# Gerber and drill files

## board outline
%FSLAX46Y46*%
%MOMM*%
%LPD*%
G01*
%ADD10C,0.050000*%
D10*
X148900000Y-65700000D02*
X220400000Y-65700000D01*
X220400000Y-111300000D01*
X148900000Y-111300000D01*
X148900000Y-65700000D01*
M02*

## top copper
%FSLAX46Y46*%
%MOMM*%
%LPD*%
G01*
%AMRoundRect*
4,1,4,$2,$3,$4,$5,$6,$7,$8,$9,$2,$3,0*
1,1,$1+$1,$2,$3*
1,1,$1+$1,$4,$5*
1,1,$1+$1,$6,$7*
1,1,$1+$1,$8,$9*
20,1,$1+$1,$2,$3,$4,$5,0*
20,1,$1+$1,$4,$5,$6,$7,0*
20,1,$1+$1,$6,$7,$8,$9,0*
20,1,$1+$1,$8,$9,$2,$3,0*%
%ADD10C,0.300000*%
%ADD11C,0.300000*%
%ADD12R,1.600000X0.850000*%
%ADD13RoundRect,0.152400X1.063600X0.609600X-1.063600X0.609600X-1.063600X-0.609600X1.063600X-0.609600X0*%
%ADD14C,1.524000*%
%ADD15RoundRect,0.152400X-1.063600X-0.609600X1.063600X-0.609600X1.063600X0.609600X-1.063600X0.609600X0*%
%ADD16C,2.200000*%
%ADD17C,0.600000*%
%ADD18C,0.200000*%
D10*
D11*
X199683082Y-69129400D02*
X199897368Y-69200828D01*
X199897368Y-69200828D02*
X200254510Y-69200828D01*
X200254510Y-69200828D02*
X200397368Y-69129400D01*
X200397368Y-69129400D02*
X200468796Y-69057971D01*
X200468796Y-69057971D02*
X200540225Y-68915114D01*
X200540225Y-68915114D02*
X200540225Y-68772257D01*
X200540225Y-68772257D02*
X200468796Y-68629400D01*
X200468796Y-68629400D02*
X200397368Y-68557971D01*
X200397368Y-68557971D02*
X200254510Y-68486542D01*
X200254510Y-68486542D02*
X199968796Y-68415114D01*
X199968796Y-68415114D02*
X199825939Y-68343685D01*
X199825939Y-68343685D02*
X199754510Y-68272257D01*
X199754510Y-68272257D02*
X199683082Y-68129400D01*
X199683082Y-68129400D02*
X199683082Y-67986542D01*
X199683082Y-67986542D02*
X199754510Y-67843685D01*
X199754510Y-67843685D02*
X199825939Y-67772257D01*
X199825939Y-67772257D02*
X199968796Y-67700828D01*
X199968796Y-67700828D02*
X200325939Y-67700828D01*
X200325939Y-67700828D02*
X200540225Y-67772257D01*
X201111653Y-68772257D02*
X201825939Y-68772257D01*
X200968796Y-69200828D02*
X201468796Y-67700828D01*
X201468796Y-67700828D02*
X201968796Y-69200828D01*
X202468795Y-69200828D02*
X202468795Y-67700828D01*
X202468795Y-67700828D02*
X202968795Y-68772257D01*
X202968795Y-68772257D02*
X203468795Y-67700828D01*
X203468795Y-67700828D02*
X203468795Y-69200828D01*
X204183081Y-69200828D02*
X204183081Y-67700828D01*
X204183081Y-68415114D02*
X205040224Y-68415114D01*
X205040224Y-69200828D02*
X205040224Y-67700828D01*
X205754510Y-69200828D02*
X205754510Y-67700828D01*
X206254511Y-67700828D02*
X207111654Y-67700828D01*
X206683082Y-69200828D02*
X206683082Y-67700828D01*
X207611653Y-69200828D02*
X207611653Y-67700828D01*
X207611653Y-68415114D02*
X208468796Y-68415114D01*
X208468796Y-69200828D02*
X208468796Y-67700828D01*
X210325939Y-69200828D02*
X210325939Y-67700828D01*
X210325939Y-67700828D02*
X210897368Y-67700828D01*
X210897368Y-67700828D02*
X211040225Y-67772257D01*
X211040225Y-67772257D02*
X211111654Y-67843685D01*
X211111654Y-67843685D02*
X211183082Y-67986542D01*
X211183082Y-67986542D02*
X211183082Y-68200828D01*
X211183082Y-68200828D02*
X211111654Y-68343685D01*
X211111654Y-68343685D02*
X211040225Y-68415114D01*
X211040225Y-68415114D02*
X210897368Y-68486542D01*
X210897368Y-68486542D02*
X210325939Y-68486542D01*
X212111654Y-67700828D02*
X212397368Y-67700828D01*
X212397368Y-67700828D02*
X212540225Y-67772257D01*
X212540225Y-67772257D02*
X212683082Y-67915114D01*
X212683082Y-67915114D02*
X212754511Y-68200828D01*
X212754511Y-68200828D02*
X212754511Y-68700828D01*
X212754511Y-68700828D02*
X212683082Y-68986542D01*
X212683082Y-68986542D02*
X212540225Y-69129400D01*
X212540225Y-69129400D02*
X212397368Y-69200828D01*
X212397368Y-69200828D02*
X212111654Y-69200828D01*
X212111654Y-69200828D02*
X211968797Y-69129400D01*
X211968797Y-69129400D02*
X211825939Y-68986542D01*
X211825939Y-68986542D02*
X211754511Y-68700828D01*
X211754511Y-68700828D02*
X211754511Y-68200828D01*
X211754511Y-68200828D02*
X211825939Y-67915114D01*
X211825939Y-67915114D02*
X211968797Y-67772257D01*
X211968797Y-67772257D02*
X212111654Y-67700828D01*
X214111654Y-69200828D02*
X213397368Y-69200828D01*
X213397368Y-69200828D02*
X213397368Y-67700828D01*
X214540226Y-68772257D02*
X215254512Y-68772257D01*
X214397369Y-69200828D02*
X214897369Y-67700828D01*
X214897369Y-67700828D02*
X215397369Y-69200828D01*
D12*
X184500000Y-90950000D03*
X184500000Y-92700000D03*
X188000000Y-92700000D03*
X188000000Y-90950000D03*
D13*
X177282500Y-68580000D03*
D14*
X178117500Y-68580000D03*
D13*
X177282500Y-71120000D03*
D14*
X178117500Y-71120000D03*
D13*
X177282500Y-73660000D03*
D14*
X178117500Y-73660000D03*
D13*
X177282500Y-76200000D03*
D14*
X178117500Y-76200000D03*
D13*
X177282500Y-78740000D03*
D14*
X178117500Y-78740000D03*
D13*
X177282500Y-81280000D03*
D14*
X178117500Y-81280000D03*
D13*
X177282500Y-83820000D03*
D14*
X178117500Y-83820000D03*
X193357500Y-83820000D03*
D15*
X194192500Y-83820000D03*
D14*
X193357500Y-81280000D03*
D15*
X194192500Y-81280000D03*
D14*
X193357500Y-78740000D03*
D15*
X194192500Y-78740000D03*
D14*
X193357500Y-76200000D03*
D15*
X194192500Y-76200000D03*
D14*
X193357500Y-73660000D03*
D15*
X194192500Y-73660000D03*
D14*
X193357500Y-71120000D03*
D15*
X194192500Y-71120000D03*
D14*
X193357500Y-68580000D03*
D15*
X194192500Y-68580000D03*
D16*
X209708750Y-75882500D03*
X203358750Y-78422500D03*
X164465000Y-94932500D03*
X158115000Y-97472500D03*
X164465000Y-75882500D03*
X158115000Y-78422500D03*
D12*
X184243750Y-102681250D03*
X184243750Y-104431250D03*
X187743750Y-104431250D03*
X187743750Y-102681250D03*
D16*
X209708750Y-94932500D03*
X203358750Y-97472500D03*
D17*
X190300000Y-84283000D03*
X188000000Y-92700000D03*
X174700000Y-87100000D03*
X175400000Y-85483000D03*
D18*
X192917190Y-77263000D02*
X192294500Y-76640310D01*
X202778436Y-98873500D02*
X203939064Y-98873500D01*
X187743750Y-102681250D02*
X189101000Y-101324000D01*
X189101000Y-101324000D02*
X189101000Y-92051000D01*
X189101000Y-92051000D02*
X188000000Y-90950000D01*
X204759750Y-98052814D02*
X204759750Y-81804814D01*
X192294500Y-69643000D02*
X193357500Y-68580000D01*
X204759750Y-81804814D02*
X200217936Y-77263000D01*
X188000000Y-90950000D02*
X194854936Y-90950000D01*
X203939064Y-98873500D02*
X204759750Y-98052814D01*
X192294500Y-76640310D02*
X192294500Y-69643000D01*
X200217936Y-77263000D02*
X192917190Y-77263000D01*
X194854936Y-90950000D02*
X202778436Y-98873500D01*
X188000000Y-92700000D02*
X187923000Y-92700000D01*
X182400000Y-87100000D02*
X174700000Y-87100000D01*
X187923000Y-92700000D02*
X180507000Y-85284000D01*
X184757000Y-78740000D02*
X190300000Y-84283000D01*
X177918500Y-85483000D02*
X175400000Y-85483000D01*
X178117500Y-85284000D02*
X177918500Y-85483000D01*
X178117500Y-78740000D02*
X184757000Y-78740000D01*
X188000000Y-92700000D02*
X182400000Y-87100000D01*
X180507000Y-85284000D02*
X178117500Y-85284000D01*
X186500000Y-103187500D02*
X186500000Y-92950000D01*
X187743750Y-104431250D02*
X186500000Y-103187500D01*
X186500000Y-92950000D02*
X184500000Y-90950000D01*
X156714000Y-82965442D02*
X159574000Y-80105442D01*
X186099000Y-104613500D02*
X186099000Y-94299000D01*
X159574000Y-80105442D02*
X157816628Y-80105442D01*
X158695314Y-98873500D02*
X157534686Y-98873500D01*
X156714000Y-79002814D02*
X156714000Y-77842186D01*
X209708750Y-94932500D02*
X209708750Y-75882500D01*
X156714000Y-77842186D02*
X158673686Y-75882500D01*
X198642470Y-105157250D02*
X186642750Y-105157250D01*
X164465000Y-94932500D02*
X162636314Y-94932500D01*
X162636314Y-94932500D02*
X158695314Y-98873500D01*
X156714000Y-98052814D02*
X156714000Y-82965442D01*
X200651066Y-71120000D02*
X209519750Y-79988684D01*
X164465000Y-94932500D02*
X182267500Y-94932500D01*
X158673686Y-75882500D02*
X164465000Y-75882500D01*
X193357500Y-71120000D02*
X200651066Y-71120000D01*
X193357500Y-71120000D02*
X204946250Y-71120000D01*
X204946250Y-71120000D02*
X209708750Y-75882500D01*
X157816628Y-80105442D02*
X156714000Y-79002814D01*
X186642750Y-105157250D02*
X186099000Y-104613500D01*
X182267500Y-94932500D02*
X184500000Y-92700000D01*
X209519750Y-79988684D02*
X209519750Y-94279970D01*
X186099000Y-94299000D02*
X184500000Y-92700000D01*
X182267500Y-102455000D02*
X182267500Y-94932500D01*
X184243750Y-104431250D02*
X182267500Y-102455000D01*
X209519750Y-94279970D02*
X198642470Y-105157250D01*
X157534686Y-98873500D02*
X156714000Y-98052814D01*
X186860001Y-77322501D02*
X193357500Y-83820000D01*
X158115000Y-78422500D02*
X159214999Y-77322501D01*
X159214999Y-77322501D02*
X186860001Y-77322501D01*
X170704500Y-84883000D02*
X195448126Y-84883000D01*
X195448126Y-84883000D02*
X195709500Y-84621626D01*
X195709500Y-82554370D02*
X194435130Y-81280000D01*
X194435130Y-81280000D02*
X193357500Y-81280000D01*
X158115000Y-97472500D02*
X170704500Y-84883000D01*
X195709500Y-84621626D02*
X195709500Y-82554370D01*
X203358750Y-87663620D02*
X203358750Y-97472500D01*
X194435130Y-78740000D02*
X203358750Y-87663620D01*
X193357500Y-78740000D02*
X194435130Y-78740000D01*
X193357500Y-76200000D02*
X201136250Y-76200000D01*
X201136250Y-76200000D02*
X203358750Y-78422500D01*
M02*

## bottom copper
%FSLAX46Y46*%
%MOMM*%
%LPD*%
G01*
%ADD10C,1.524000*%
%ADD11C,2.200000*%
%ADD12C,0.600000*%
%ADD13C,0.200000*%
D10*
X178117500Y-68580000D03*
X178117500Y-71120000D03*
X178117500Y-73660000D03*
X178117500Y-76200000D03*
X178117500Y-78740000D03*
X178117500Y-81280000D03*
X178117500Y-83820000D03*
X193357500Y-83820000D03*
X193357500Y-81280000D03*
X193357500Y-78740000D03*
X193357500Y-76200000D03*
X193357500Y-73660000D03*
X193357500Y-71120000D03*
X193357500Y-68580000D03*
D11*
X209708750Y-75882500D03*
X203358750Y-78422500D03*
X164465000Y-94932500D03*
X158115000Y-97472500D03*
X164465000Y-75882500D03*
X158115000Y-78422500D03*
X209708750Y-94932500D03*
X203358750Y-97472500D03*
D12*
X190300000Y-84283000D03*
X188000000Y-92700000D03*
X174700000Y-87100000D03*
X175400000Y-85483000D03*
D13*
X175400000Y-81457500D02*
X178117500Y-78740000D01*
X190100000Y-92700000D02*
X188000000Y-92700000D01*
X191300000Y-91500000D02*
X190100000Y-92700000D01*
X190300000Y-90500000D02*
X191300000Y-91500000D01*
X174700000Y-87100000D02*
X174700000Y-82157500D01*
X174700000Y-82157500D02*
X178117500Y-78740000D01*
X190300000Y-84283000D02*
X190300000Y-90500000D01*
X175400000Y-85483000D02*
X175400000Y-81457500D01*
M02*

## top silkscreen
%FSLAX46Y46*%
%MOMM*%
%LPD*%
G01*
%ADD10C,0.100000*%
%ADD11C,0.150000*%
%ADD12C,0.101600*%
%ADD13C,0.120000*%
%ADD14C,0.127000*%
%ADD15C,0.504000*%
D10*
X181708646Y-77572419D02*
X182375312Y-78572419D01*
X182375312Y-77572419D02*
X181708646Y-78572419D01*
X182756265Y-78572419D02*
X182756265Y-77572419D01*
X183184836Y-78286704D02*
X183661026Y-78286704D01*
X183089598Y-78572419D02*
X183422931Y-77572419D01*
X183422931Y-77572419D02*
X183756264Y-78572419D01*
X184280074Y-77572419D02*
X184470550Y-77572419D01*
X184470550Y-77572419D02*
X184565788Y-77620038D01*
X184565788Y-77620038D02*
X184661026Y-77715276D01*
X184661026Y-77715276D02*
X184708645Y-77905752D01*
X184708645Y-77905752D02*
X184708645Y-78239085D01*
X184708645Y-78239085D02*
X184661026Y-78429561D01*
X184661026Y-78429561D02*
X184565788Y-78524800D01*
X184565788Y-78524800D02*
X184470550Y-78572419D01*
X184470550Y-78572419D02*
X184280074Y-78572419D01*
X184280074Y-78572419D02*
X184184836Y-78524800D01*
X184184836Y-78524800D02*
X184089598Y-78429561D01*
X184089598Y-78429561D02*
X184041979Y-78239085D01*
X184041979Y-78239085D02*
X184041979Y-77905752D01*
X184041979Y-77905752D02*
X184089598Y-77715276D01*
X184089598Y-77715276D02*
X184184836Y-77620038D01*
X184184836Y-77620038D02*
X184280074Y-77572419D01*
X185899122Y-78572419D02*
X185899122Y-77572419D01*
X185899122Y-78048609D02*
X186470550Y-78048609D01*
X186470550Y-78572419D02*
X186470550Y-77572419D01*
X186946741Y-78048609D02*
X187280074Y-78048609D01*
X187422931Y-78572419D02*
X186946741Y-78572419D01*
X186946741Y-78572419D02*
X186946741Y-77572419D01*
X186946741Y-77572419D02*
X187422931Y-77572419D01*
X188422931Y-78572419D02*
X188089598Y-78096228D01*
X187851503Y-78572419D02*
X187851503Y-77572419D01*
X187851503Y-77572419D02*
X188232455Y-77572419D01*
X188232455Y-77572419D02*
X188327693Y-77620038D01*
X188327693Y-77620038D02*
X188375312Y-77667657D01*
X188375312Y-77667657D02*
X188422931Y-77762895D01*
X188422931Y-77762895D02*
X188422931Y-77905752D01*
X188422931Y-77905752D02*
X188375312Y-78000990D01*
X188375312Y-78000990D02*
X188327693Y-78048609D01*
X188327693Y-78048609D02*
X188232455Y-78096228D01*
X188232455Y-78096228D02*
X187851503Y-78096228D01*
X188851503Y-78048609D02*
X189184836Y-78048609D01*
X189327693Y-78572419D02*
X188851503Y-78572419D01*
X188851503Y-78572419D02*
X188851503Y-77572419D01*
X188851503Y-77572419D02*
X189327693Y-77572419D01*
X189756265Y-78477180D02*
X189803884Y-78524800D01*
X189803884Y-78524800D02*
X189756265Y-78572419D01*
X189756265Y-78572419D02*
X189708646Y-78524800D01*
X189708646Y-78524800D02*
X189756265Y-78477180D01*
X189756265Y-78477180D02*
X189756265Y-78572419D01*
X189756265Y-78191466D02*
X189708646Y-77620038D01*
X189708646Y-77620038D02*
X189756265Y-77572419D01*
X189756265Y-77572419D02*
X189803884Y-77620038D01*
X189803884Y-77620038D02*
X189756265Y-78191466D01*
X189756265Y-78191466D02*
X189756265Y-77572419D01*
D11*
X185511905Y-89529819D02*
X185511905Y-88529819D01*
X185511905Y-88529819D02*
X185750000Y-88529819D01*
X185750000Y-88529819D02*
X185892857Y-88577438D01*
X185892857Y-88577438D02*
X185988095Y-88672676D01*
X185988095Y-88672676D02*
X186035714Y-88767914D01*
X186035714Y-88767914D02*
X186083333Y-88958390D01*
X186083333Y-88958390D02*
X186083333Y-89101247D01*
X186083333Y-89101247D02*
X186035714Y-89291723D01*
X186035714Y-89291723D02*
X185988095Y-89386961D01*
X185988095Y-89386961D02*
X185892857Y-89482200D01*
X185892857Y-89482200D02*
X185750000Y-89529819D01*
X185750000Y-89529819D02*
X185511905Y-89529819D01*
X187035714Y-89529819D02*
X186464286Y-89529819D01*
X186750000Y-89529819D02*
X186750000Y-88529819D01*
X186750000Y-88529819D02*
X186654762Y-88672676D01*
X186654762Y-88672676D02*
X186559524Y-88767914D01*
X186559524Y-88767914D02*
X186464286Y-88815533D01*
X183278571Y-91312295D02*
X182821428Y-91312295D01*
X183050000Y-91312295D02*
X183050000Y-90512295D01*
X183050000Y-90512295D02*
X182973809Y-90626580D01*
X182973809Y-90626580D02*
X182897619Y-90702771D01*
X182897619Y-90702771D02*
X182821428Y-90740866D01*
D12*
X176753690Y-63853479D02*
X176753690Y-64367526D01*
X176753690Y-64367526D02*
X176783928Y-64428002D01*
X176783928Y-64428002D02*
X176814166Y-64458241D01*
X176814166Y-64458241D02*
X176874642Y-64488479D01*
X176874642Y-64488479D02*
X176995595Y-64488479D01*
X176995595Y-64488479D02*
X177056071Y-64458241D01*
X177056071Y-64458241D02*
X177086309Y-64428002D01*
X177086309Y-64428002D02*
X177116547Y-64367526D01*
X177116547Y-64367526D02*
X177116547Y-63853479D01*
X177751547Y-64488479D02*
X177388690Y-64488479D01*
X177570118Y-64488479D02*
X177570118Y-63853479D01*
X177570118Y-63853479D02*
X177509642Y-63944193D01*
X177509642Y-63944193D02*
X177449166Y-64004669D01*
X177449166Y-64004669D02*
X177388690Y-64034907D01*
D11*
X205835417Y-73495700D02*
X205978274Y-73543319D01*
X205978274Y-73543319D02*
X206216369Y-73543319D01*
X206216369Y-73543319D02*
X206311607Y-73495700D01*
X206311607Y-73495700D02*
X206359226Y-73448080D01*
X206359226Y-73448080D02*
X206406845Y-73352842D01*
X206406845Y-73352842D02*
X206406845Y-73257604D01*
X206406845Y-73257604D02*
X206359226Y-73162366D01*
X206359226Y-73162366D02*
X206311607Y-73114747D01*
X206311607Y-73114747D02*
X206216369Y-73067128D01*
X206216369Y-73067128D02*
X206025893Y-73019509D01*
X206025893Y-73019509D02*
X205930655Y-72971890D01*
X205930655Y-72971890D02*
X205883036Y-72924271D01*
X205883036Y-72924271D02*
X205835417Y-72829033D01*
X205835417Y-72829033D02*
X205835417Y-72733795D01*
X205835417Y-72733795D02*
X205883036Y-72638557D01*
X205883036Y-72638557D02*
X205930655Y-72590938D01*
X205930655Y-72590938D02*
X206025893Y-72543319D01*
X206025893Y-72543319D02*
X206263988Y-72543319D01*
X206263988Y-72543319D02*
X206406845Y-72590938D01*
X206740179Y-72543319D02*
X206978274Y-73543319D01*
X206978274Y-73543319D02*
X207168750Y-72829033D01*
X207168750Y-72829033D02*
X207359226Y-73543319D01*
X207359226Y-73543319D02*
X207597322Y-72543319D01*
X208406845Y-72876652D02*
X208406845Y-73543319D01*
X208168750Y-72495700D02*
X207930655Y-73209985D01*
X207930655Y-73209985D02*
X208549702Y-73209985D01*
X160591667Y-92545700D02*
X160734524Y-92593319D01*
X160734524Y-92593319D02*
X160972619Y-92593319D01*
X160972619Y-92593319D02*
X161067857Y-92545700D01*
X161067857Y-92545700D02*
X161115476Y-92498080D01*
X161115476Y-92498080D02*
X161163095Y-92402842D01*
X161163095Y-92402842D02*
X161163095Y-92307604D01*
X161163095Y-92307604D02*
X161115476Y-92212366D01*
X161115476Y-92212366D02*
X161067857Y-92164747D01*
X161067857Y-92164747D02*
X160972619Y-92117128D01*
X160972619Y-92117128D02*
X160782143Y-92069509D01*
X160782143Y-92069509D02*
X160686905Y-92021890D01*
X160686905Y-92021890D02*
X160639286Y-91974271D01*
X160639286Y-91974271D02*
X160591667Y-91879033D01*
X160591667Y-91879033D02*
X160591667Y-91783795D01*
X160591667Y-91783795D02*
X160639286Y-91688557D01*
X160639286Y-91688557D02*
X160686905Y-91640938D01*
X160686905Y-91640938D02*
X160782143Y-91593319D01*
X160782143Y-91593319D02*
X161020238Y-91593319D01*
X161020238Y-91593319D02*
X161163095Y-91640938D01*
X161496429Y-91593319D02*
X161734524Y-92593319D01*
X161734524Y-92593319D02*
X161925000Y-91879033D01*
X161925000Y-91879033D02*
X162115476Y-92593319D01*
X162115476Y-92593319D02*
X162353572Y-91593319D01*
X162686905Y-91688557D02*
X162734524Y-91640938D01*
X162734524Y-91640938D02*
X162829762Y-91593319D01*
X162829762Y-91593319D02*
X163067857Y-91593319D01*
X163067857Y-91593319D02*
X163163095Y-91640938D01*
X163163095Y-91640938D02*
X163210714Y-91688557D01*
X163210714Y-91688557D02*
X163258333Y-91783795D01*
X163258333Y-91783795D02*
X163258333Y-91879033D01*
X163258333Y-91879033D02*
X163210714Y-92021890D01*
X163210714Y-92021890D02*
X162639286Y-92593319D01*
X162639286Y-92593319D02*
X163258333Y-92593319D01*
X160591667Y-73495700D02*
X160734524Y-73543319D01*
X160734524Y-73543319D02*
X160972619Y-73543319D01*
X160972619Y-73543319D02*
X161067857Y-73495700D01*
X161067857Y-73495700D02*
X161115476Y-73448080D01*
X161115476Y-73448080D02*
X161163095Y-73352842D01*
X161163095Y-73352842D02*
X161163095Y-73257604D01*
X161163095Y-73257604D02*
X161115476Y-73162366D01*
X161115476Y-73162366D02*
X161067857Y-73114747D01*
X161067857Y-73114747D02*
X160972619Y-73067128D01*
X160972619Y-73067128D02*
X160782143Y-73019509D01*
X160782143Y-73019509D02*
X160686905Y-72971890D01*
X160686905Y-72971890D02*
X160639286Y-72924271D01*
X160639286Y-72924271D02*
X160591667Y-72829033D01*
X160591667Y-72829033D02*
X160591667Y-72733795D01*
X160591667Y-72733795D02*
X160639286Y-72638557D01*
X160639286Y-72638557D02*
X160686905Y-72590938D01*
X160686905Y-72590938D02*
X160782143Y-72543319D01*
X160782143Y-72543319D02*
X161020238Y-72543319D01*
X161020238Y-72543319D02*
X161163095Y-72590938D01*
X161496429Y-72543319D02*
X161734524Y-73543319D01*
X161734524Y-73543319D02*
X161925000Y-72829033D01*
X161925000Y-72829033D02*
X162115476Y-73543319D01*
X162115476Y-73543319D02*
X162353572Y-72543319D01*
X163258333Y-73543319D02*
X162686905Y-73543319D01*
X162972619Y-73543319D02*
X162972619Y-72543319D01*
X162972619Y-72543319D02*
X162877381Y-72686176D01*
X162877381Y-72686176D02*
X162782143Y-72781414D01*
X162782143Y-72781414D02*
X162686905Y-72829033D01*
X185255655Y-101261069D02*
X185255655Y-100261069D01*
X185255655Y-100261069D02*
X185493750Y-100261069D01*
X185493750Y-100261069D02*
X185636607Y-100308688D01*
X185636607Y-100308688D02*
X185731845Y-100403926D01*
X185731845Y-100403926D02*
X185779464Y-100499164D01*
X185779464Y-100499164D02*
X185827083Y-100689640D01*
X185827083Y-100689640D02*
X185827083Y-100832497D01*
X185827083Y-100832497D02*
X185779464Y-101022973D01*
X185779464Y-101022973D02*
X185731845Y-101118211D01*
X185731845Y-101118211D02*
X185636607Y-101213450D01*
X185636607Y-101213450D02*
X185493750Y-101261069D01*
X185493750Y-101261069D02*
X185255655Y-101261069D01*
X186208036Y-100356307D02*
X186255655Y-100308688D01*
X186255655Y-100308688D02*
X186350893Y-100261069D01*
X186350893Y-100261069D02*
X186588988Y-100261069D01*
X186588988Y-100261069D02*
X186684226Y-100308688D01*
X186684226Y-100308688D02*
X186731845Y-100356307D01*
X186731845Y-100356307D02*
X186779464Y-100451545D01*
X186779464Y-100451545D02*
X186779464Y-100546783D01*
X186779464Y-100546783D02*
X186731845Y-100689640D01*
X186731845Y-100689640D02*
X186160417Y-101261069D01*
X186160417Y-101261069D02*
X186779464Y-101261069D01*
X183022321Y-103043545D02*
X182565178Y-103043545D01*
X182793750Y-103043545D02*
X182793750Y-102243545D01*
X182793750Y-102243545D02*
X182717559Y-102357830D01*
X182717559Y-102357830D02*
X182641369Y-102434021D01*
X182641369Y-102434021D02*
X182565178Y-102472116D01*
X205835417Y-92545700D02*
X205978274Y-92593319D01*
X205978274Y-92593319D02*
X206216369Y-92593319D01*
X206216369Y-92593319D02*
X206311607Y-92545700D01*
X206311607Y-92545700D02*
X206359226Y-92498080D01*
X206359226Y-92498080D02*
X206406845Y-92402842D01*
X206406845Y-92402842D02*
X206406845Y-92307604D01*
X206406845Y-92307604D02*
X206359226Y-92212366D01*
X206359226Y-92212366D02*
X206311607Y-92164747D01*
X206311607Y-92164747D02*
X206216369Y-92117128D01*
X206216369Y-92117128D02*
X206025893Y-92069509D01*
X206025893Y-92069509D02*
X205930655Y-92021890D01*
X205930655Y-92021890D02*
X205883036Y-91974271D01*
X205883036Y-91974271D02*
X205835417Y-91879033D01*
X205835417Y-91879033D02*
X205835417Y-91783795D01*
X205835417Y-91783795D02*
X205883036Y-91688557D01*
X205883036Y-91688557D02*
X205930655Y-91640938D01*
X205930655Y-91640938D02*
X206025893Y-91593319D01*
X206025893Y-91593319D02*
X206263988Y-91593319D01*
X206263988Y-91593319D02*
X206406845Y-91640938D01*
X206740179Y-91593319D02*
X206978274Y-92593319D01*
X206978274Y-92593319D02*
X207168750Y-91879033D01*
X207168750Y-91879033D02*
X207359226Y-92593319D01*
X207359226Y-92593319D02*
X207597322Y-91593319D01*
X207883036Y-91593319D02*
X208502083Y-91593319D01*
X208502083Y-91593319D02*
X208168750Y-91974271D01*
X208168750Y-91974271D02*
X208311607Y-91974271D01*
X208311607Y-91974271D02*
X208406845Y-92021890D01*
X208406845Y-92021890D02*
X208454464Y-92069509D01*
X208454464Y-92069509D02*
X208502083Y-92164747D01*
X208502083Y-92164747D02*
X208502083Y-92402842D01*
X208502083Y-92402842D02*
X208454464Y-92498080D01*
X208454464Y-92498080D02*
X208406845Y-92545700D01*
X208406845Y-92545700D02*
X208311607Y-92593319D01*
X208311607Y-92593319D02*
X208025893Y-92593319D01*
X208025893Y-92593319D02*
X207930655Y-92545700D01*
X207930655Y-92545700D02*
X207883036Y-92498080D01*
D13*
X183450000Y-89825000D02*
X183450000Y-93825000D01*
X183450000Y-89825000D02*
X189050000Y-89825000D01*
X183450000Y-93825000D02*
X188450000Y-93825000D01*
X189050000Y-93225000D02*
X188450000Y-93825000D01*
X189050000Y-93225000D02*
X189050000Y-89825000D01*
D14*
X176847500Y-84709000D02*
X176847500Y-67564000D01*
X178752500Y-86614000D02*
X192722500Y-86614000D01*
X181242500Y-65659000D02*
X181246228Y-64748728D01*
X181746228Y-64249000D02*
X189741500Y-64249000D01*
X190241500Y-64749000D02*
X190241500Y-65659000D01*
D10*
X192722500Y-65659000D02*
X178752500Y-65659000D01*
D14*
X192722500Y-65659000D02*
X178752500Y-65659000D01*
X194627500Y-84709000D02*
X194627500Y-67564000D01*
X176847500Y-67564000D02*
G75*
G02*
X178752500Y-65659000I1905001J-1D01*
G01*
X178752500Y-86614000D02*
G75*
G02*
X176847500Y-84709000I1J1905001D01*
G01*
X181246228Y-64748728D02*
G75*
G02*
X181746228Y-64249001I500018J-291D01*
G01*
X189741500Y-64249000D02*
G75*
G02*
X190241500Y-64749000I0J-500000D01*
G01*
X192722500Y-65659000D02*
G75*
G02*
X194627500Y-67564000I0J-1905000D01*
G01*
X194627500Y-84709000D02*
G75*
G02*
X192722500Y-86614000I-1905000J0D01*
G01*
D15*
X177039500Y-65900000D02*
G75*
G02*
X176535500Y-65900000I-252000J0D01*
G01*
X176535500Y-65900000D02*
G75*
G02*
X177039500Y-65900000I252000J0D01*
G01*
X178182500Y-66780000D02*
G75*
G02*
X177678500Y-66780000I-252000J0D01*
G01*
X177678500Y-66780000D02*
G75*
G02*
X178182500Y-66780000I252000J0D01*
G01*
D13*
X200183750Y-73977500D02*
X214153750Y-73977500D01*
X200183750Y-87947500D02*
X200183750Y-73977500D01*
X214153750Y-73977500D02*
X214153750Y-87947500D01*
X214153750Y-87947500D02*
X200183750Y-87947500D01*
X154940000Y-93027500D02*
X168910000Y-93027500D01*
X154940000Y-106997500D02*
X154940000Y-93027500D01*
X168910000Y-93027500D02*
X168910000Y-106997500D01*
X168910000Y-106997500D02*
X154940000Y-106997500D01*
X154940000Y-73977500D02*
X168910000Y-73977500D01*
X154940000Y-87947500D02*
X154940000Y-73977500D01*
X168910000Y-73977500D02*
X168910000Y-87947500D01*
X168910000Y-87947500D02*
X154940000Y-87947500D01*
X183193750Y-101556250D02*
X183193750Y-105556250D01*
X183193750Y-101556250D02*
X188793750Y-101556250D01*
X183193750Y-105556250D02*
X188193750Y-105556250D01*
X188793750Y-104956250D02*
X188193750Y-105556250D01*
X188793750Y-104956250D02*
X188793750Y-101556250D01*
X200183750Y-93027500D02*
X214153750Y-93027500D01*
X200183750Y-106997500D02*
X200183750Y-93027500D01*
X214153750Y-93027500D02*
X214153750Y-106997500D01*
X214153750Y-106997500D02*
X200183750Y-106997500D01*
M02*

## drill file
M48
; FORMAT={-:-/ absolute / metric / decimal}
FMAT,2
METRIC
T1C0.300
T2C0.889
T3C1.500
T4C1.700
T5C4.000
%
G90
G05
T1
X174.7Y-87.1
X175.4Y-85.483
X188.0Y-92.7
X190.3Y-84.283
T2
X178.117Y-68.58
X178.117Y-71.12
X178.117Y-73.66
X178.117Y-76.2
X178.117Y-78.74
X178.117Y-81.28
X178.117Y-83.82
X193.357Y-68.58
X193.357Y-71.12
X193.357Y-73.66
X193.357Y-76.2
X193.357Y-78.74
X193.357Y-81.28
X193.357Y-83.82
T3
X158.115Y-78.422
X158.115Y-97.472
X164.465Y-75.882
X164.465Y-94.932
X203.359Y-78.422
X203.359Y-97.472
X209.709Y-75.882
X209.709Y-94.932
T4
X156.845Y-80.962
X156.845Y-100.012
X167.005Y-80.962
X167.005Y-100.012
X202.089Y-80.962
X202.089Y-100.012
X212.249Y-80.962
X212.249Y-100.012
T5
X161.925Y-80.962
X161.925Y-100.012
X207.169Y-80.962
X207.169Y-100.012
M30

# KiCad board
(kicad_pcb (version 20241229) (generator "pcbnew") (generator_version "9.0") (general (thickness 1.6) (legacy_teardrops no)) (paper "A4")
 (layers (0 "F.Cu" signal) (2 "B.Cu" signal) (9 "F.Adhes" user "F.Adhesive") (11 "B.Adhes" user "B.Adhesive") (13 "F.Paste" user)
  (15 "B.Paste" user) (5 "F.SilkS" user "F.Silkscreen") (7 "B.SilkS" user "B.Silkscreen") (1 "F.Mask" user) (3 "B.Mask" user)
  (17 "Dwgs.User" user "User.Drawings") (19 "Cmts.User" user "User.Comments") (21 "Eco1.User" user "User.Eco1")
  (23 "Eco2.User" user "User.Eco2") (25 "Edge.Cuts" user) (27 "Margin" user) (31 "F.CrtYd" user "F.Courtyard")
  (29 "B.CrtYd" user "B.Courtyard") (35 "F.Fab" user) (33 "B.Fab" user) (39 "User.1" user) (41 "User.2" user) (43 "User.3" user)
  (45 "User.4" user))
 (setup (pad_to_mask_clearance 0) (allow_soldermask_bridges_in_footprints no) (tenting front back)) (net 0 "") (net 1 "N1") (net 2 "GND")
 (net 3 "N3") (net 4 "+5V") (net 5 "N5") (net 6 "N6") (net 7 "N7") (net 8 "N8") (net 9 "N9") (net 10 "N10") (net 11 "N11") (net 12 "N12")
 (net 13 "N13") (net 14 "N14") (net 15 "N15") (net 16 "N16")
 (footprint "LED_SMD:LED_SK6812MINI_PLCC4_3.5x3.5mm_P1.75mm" (layer "F.Cu") (at 186.25 91.825)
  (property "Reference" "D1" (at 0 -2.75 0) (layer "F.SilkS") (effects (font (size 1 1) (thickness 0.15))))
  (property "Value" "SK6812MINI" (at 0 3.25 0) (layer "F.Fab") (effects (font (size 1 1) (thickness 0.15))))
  (fp_line (start -2.8 -2) (end -2.8 2) (stroke (width 0.12) (type default)) (layer "F.SilkS"))
  (fp_line (start -2.8 -2) (end 2.8 -2) (stroke (width 0.12) (type solid)) (layer "F.SilkS"))
  (fp_line (start -2.8 2) (end 2.2 2) (stroke (width 0.12) (type solid)) (layer "F.SilkS"))
  (fp_line (start 2.8 1.4) (end 2.2 2) (stroke (width 0.12) (type default)) (layer "F.SilkS"))
  (fp_line (start 2.8 1.4) (end 2.8 -2) (stroke (width 0.12) (type solid)) (layer "F.SilkS"))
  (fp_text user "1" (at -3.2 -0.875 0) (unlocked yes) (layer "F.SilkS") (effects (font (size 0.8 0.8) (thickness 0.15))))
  (pad "1" smd rect (at -1.75 -0.875) (size 1.6 0.85) (layers "F.Cu" "F.Mask" "F.Paste") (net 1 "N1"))
  (pad "2" smd rect (at -1.75 0.875) (size 1.6 0.85) (layers "F.Cu" "F.Mask" "F.Paste") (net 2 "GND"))
  (pad "3" smd rect (at 1.75 0.875) (size 1.6 0.85) (layers "F.Cu" "F.Mask" "F.Paste") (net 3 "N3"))
  (pad "4" smd rect (at 1.75 -0.875) (size 1.6 0.85) (layers "F.Cu" "F.Mask" "F.Paste") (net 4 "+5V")))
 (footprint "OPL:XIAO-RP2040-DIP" (layer "F.Cu") (at 185.7375 76.2)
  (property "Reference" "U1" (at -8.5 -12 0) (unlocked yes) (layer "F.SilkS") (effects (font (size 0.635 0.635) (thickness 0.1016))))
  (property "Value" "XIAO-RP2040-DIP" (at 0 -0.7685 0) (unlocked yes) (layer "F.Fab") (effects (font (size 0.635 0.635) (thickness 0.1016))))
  (fp_line (start -8.89 8.509) (end -8.89 -8.636) (stroke (width 0.127) (type solid)) (layer "F.SilkS"))
  (fp_line (start -6.985 10.414) (end 6.985 10.414) (stroke (width 0.127) (type solid)) (layer "F.SilkS"))
  (fp_line (start -4.495 -10.541) (end -4.491272 -11.451272) (stroke (width 0.127) (type solid)) (layer "F.SilkS"))
  (fp_line (start -3.991272 -11.951) (end 4.004 -11.951) (stroke (width 0.127) (type solid)) (layer "F.SilkS"))
  (fp_line (start 4.504 -11.451) (end 4.504 -10.541) (stroke (width 0.127) (type solid)) (layer "F.SilkS"))
  (fp_line (start 6.985 -10.541) (end -6.985 -10.541) (stroke (width 0.1) (type solid)) (layer "F.SilkS"))
  (fp_line (start 6.985 -10.541) (end -6.985 -10.541) (stroke (width 0.127) (type solid)) (layer "F.SilkS"))
  (fp_line (start 8.89 8.509) (end 8.89 -8.636) (stroke (width 0.127) (type solid)) (layer "F.SilkS"))
  (fp_arc (start -8.89 -8.636) (mid -8.332038 -9.983038) (end -6.985 -10.541) (stroke (width 0.127) (type solid)) (layer "F.SilkS"))
  (fp_arc (start -6.985 10.414) (mid -8.332038 9.856038) (end -8.89 8.509) (stroke (width 0.127) (type solid)) (layer "F.SilkS"))
  (fp_arc (start -4.491272 -11.451272) (mid -4.344728 -11.80464) (end -3.991272 -11.951) (stroke (width 0.127) (type default))
   (layer "F.SilkS"))
  (fp_arc (start 4.004 -11.951) (mid 4.357553 -11.804553) (end 4.504 -11.451) (stroke (width 0.127) (type default)) (layer "F.SilkS"))
  (fp_arc (start 6.985 -10.541) (mid 8.332038 -9.983038) (end 8.89 -8.636) (stroke (width 0.127) (type solid)) (layer "F.SilkS"))
  (fp_arc (start 8.89 8.509) (mid 8.332038 9.856038) (end 6.985 10.414) (stroke (width 0.127) (type solid)) (layer "F.SilkS"))
  (fp_circle (center -8.95 -10.3) (end -8.95 -10.554) (stroke (width 0.5) (type solid)) (fill yes) (layer "F.SilkS"))
  (fp_circle (center -7.807 -9.42) (end -7.807 -9.674) (stroke (width 0.5) (type solid)) (fill yes) (layer "F.SilkS"))
  (pad "1" smd roundrect (at -8.455 -7.62 180) (size 2.432 1.524) (layers "F.Cu" "F.Mask") (roundrect_rratio 0.1) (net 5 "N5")
   (thermal_bridge_angle 45))
  (pad "1" thru_hole circle (at -7.62 -7.62 180) (size 1.524 1.524) (drill 0.889) (layers "*.Cu" "*.Mask") (remove_unused_layers no)
   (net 5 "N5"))
  (pad "2" smd roundrect (at -8.455 -5.08 180) (size 2.432 1.524) (layers "F.Cu" "F.Mask") (roundrect_rratio 0.1) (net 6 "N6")
   (thermal_bridge_angle 45))
  (pad "2" thru_hole circle (at -7.62 -5.08 180) (size 1.524 1.524) (drill 0.889) (layers "*.Cu" "*.Mask") (remove_unused_layers no)
   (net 6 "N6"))
  (pad "3" smd roundrect (at -8.455 -2.54 180) (size 2.432 1.524) (layers "F.Cu" "F.Mask") (roundrect_rratio 0.1) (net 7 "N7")
   (thermal_bridge_angle 45))
  (pad "3" thru_hole circle (at -7.62 -2.54 180) (size 1.524 1.524) (drill 0.889) (layers "*.Cu" "*.Mask") (remove_unused_layers no)
   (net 7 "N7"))
  (pad "4" smd roundrect (at -8.455 0 180) (size 2.432 1.524) (layers "F.Cu" "F.Mask") (roundrect_rratio 0.1) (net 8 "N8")
   (thermal_bridge_angle 45))
  (pad "4" thru_hole circle (at -7.62 0 180) (size 1.524 1.524) (drill 0.889) (layers "*.Cu" "*.Mask") (remove_unused_layers no)
   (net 8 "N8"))
  (pad "5" smd roundrect (at -8.455 2.54 180) (size 2.432 1.524) (layers "F.Cu" "F.Mask") (roundrect_rratio 0.1) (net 3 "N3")
   (thermal_bridge_angle 45))
  (pad "5" thru_hole circle (at -7.62 2.54 180) (size 1.524 1.524) (drill 0.889) (layers "*.Cu" "*.Mask") (remove_unused_layers no)
   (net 3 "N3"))
  (pad "6" smd roundrect (at -8.455 5.08 180) (size 2.432 1.524) (layers "F.Cu" "F.Mask") (roundrect_rratio 0.1) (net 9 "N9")
   (thermal_bridge_angle 45))
  (pad "6" thru_hole circle (at -7.62 5.08 180) (size 1.524 1.524) (drill 0.889) (layers "*.Cu" "*.Mask") (remove_unused_layers no)
   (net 9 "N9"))
  (pad "7" smd roundrect (at -8.455 7.62 180) (size 2.432 1.524) (layers "F.Cu" "F.Mask") (roundrect_rratio 0.1) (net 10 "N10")
   (thermal_bridge_angle 45))
  (pad "7" thru_hole circle (at -7.62 7.62 180) (size 1.524 1.524) (drill 0.889) (layers "*.Cu" "*.Mask") (remove_unused_layers no)
   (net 10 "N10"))
  (pad "8" thru_hole circle (at 7.62 7.62) (size 1.524 1.524) (drill 0.889) (layers "*.Cu" "*.Mask") (remove_unused_layers no)
   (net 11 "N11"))
  (pad "8" smd roundrect (at 8.455 7.62) (size 2.432 1.524) (layers "F.Cu" "F.Mask") (roundrect_rratio 0.1) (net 11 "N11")
   (thermal_bridge_angle 45))
  (pad "9" thru_hole circle (at 7.62 5.08) (size 1.524 1.524) (drill 0.889) (layers "*.Cu" "*.Mask") (remove_unused_layers no)
   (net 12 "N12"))
  (pad "9" smd roundrect (at 8.455 5.08) (size 2.432 1.524) (layers "F.Cu" "F.Mask") (roundrect_rratio 0.1) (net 12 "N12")
   (thermal_bridge_angle 45))
  (pad "10" thru_hole circle (at 7.62 2.54) (size 1.524 1.524) (drill 0.889) (layers "*.Cu" "*.Mask") (remove_unused_layers no)
   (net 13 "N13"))
  (pad "10" smd roundrect (at 8.455 2.54) (size 2.432 1.524) (layers "F.Cu" "F.Mask") (roundrect_rratio 0.1) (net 13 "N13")
   (thermal_bridge_angle 45))
  (pad "11" thru_hole circle (at 7.62 0) (size 1.524 1.524) (drill 0.889) (layers "*.Cu" "*.Mask") (remove_unused_layers no) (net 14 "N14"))
  (pad "11" smd roundrect (at 8.455 0) (size 2.432 1.524) (layers "F.Cu" "F.Mask") (roundrect_rratio 0.1) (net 14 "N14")
   (thermal_bridge_angle 45))
  (pad "12" thru_hole circle (at 7.62 -2.54) (size 1.524 1.524) (drill 0.889) (layers "*.Cu" "*.Mask") (remove_unused_layers no)
   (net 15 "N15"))
  (pad "12" smd roundrect (at 8.455 -2.54) (size 2.432 1.524) (layers "F.Cu" "F.Mask") (roundrect_rratio 0.1) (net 15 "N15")
   (thermal_bridge_angle 45))
  (pad "13" thru_hole circle (at 7.62 -5.08) (size 1.524 1.524) (drill 0.889) (layers "*.Cu" "*.Mask") (remove_unused_layers no)
   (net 2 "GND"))
  (pad "13" smd roundrect (at 8.455 -5.08) (size 2.432 1.524) (layers "F.Cu" "F.Mask") (roundrect_rratio 0.1) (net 2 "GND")
   (thermal_bridge_angle 45))
  (pad "14" thru_hole circle (at 7.62 -7.62) (size 1.524 1.524) (drill 0.889) (layers "*.Cu" "*.Mask") (remove_unused_layers no)
   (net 4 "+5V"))
  (pad "14" smd roundrect (at 8.455 -7.62) (size 2.432 1.524) (layers "F.Cu" "F.Mask") (roundrect_rratio 0.1) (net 4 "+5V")
   (thermal_bridge_angle 45)))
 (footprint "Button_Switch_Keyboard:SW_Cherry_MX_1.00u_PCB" (layer "F.Cu") (at 209.70875 75.8825)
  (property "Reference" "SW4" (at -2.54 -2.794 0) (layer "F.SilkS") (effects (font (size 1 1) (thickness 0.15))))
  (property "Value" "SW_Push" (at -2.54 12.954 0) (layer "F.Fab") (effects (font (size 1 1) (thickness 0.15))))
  (fp_line (start -9.525 -1.905) (end 4.445 -1.905) (stroke (width 0.12) (type solid)) (layer "F.SilkS"))
  (fp_line (start -9.525 12.065) (end -9.525 -1.905) (stroke (width 0.12) (type solid)) (layer "F.SilkS"))
  (fp_line (start 4.445 -1.905) (end 4.445 12.065) (stroke (width 0.12) (type solid)) (layer "F.SilkS"))
  (fp_line (start 4.445 12.065) (end -9.525 12.065) (stroke (width 0.12) (type solid)) (layer "F.SilkS"))
  (pad "" np_thru_hole circle (at -7.62 5.08) (size 1.7 1.7) (drill 1.7) (layers "*.Cu" "*.Mask"))
  (pad "" np_thru_hole circle (at -2.54 5.08) (size 4 4) (drill 4) (layers "*.Cu" "*.Mask"))
  (pad "" np_thru_hole circle (at 2.54 5.08) (size 1.7 1.7) (drill 1.7) (layers "*.Cu" "*.Mask"))
  (pad "1" thru_hole circle (at 0 0) (size 2.2 2.2) (drill 1.5) (layers "*.Cu" "*.Mask") (remove_unused_layers no) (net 2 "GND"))
  (pad "2" thru_hole circle (at -6.35 2.54) (size 2.2 2.2) (drill 1.5) (layers "*.Cu" "*.Mask") (remove_unused_layers no) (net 14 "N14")))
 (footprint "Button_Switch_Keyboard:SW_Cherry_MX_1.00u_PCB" (layer "F.Cu") (at 164.465 94.9325)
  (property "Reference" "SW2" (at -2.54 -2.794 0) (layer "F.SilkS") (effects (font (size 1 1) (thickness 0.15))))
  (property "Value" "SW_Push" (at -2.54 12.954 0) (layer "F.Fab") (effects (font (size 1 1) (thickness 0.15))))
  (fp_line (start -9.525 -1.905) (end 4.445 -1.905) (stroke (width 0.12) (type solid)) (layer "F.SilkS"))
  (fp_line (start -9.525 12.065) (end -9.525 -1.905) (stroke (width 0.12) (type solid)) (layer "F.SilkS"))
  (fp_line (start 4.445 -1.905) (end 4.445 12.065) (stroke (width 0.12) (type solid)) (layer "F.SilkS"))
  (fp_line (start 4.445 12.065) (end -9.525 12.065) (stroke (width 0.12) (type solid)) (layer "F.SilkS"))
  (pad "" np_thru_hole circle (at -7.62 5.08) (size 1.7 1.7) (drill 1.7) (layers "*.Cu" "*.Mask"))
  (pad "" np_thru_hole circle (at -2.54 5.08) (size 4 4) (drill 4) (layers "*.Cu" "*.Mask"))
  (pad "" np_thru_hole circle (at 2.54 5.08) (size 1.7 1.7) (drill 1.7) (layers "*.Cu" "*.Mask"))
  (pad "1" thru_hole circle (at 0 0) (size 2.2 2.2) (drill 1.5) (layers "*.Cu" "*.Mask") (remove_unused_layers no) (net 2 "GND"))
  (pad "2" thru_hole circle (at -6.35 2.54) (size 2.2 2.2) (drill 1.5) (layers "*.Cu" "*.Mask") (remove_unused_layers no) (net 12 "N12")))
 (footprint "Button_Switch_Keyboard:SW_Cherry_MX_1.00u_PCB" (layer "F.Cu") (at 164.465 75.8825)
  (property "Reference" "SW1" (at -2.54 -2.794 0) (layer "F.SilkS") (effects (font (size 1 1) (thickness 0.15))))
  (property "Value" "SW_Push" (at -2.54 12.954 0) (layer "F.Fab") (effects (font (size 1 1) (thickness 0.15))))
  (fp_line (start -9.525 -1.905) (end 4.445 -1.905) (stroke (width 0.12) (type solid)) (layer "F.SilkS"))
  (fp_line (start -9.525 12.065) (end -9.525 -1.905) (stroke (width 0.12) (type solid)) (layer "F.SilkS"))
  (fp_line (start 4.445 -1.905) (end 4.445 12.065) (stroke (width 0.12) (type solid)) (layer "F.SilkS"))
  (fp_line (start 4.445 12.065) (end -9.525 12.065) (stroke (width 0.12) (type solid)) (layer "F.SilkS"))
  (pad "" np_thru_hole circle (at -7.62 5.08) (size 1.7 1.7) (drill 1.7) (layers "*.Cu" "*.Mask"))
  (pad "" np_thru_hole circle (at -2.54 5.08) (size 4 4) (drill 4) (layers "*.Cu" "*.Mask"))
  (pad "" np_thru_hole circle (at 2.54 5.08) (size 1.7 1.7) (drill 1.7) (layers "*.Cu" "*.Mask"))
  (pad "1" thru_hole circle (at 0 0) (size 2.2 2.2) (drill 1.5) (layers "*.Cu" "*.Mask") (remove_unused_layers no) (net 2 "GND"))
  (pad "2" thru_hole circle (at -6.35 2.54) (size 2.2 2.2) (drill 1.5) (layers "*.Cu" "*.Mask") (remove_unused_layers no) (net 11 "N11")))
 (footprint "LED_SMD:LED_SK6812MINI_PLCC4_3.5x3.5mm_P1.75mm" (layer "F.Cu") (at 185.99375 103.55625)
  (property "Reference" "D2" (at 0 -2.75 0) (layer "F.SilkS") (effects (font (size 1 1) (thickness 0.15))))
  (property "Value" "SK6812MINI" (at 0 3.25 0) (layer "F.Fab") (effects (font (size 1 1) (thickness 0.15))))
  (fp_line (start -2.8 -2) (end -2.8 2) (stroke (width 0.12) (type default)) (layer "F.SilkS"))
  (fp_line (start -2.8 -2) (end 2.8 -2) (stroke (width 0.12) (type solid)) (layer "F.SilkS"))
  (fp_line (start -2.8 2) (end 2.2 2) (stroke (width 0.12) (type solid)) (layer "F.SilkS"))
  (fp_line (start 2.8 1.4) (end 2.2 2) (stroke (width 0.12) (type default)) (layer "F.SilkS"))
  (fp_line (start 2.8 1.4) (end 2.8 -2) (stroke (width 0.12) (type solid)) (layer "F.SilkS"))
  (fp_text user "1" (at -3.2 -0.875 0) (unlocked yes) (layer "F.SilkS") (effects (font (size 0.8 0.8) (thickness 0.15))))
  (pad "1" smd rect (at -1.75 -0.875) (size 1.6 0.85) (layers "F.Cu" "F.Mask" "F.Paste") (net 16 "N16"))
  (pad "2" smd rect (at -1.75 0.875) (size 1.6 0.85) (layers "F.Cu" "F.Mask" "F.Paste") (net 2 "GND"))
  (pad "3" smd rect (at 1.75 0.875) (size 1.6 0.85) (layers "F.Cu" "F.Mask" "F.Paste") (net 1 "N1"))
  (pad "4" smd rect (at 1.75 -0.875) (size 1.6 0.85) (layers "F.Cu" "F.Mask" "F.Paste") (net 4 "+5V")))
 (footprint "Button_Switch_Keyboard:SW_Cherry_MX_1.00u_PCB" (layer "F.Cu") (at 209.70875 94.9325)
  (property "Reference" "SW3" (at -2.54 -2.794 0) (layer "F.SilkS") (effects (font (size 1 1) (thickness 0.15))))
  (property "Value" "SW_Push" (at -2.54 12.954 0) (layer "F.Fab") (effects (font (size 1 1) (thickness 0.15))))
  (fp_line (start -9.525 -1.905) (end 4.445 -1.905) (stroke (width 0.12) (type solid)) (layer "F.SilkS"))
  (fp_line (start -9.525 12.065) (end -9.525 -1.905) (stroke (width 0.12) (type solid)) (layer "F.SilkS"))
  (fp_line (start 4.445 -1.905) (end 4.445 12.065) (stroke (width 0.12) (type solid)) (layer "F.SilkS"))
  (fp_line (start 4.445 12.065) (end -9.525 12.065) (stroke (width 0.12) (type solid)) (layer "F.SilkS"))
  (pad "" np_thru_hole circle (at -7.62 5.08) (size 1.7 1.7) (drill 1.7) (layers "*.Cu" "*.Mask"))
  (pad "" np_thru_hole circle (at -2.54 5.08) (size 4 4) (drill 4) (layers "*.Cu" "*.Mask"))
  (pad "" np_thru_hole circle (at 2.54 5.08) (size 1.7 1.7) (drill 1.7) (layers "*.Cu" "*.Mask"))
  (pad "1" thru_hole circle (at 0 0) (size 2.2 2.2) (drill 1.5) (layers "*.Cu" "*.Mask") (remove_unused_layers no) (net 2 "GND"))
  (pad "2" thru_hole circle (at -6.35 2.54) (size 2.2 2.2) (drill 1.5) (layers "*.Cu" "*.Mask") (remove_unused_layers no) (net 13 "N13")))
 (gr_rect (start 148.9 65.7) (end 220.4 111.3) (stroke (width 0.05) (type default)) (fill no) (layer "Edge.Cuts"))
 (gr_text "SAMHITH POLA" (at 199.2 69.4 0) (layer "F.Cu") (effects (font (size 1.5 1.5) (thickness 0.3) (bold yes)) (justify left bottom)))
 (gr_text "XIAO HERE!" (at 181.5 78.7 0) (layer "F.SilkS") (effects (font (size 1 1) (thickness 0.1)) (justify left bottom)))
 (segment (start 192.91719 77.263) (end 192.2945 76.64031) (width 0.2) (layer "F.Cu") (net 4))
 (segment (start 202.778436 98.8735) (end 203.939064 98.8735) (width 0.2) (layer "F.Cu") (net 4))
 (segment (start 187.74375 102.68125) (end 189.101 101.324) (width 0.2) (layer "F.Cu") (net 4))
 (segment (start 189.101 101.324) (end 189.101 92.051) (width 0.2) (layer "F.Cu") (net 4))
 (segment (start 189.101 92.051) (end 188 90.95) (width 0.2) (layer "F.Cu") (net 4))
 (segment (start 204.75975 98.052814) (end 204.75975 81.804814) (width 0.2) (layer "F.Cu") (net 4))
 (segment (start 192.2945 69.643) (end 193.3575 68.58) (width 0.2) (layer "F.Cu") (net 4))
 (segment (start 204.75975 81.804814) (end 200.217936 77.263) (width 0.2) (layer "F.Cu") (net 4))
 (segment (start 188 90.95) (end 194.854936 90.95) (width 0.2) (layer "F.Cu") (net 4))
 (segment (start 203.939064 98.8735) (end 204.75975 98.052814) (width 0.2) (layer "F.Cu") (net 4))
 (segment (start 192.2945 76.64031) (end 192.2945 69.643) (width 0.2) (layer "F.Cu") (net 4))
 (segment (start 200.217936 77.263) (end 192.91719 77.263) (width 0.2) (layer "F.Cu") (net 4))
 (segment (start 194.854936 90.95) (end 202.778436 98.8735) (width 0.2) (layer "F.Cu") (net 4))
 (segment (start 188 92.7) (end 187.923 92.7) (width 0.2) (layer "F.Cu") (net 3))
 (segment (start 182.4 87.1) (end 174.7 87.1) (width 0.2) (layer "F.Cu") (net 3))
 (segment (start 187.923 92.7) (end 180.507 85.284) (width 0.2) (layer "F.Cu") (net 3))
 (segment (start 184.757 78.74) (end 190.3 84.283) (width 0.2) (layer "F.Cu") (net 3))
 (segment (start 177.9185 85.483) (end 175.4 85.483) (width 0.2) (layer "F.Cu") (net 3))
 (segment (start 178.1175 85.284) (end 177.9185 85.483) (width 0.2) (layer "F.Cu") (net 3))
 (segment (start 178.1175 78.74) (end 184.757 78.74) (width 0.2) (layer "F.Cu") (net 3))
 (segment (start 188 92.7) (end 182.4 87.1) (width 0.2) (layer "F.Cu") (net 3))
 (segment (start 180.507 85.284) (end 178.1175 85.284) (width 0.2) (layer "F.Cu") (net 3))
 (via (at 190.3 84.283) (size 0.6) (drill 0.3) (layers "F.Cu" "B.Cu") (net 3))
 (via (at 188 92.7) (size 0.6) (drill 0.3) (layers "F.Cu" "B.Cu") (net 3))
 (via (at 174.7 87.1) (size 0.6) (drill 0.3) (layers "F.Cu" "B.Cu") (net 3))
 (via (at 175.4 85.483) (size 0.6) (drill 0.3) (layers "F.Cu" "B.Cu") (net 3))
 (segment (start 175.4 81.4575) (end 178.1175 78.74) (width 0.2) (layer "B.Cu") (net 3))
 (segment (start 190.1 92.7) (end 188 92.7) (width 0.2) (layer "B.Cu") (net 3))
 (segment (start 191.3 91.5) (end 190.1 92.7) (width 0.2) (layer "B.Cu") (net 3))
 (segment (start 190.3 90.5) (end 191.3 91.5) (width 0.2) (layer "B.Cu") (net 3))
 (segment (start 174.7 87.1) (end 174.7 82.1575) (width 0.2) (layer "B.Cu") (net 3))
 (segment (start 174.7 82.1575) (end 178.1175 78.74) (width 0.2) (layer "B.Cu") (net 3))
 (segment (start 190.3 84.283) (end 190.3 90.5) (width 0.2) (layer "B.Cu") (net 3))
 (segment (start 175.4 85.483) (end 175.4 81.4575) (width 0.2) (layer "B.Cu") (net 3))
 (segment (start 186.5 103.1875) (end 186.5 92.95) (width 0.2) (layer "F.Cu") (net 1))
 (segment (start 187.74375 104.43125) (end 186.5 103.1875) (width 0.2) (layer "F.Cu") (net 1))
 (segment (start 186.5 92.95) (end 184.5 90.95) (width 0.2) (layer "F.Cu") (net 1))
 (segment (start 156.714 82.965442) (end 159.574 80.105442) (width 0.2) (layer "F.Cu") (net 2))
 (segment (start 186.099 104.6135) (end 186.099 94.299) (width 0.2) (layer "F.Cu") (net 2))
 (segment (start 159.574 80.105442) (end 157.816628 80.105442) (width 0.2) (layer "F.Cu") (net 2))
 (segment (start 158.695314 98.8735) (end 157.534686 98.8735) (width 0.2) (layer "F.Cu") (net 2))
 (segment (start 156.714 79.002814) (end 156.714 77.842186) (width 0.2) (layer "F.Cu") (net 2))
 (segment (start 209.70875 94.9325) (end 209.70875 75.8825) (width 0.2) (layer "F.Cu") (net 2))
 (segment (start 156.714 77.842186) (end 158.673686 75.8825) (width 0.2) (layer "F.Cu") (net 2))
 (segment (start 198.64247 105.15725) (end 186.64275 105.15725) (width 0.2) (layer "F.Cu") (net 2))
 (segment (start 164.465 94.9325) (end 162.636314 94.9325) (width 0.2) (layer "F.Cu") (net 2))
 (segment (start 162.636314 94.9325) (end 158.695314 98.8735) (width 0.2) (layer "F.Cu") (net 2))
 (segment (start 156.714 98.052814) (end 156.714 82.965442) (width 0.2) (layer "F.Cu") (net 2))
 (segment (start 200.651066 71.12) (end 209.51975 79.988684) (width 0.2) (layer "F.Cu") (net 2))
 (segment (start 164.465 94.9325) (end 182.2675 94.9325) (width 0.2) (layer "F.Cu") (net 2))
 (segment (start 158.673686 75.8825) (end 164.465 75.8825) (width 0.2) (layer "F.Cu") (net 2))
 (segment (start 193.3575 71.12) (end 200.651066 71.12) (width 0.2) (layer "F.Cu") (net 2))
 (segment (start 193.3575 71.12) (end 204.94625 71.12) (width 0.2) (layer "F.Cu") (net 2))
 (segment (start 204.94625 71.12) (end 209.70875 75.8825) (width 0.2) (layer "F.Cu") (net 2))
 (segment (start 157.816628 80.105442) (end 156.714 79.002814) (width 0.2) (layer "F.Cu") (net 2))
 (segment (start 186.64275 105.15725) (end 186.099 104.6135) (width 0.2) (layer "F.Cu") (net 2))
 (segment (start 182.2675 94.9325) (end 184.5 92.7) (width 0.2) (layer "F.Cu") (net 2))
 (segment (start 209.51975 79.988684) (end 209.51975 94.27997) (width 0.2) (layer "F.Cu") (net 2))
 (segment (start 186.099 94.299) (end 184.5 92.7) (width 0.2) (layer "F.Cu") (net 2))
 (segment (start 182.2675 102.455) (end 182.2675 94.9325) (width 0.2) (layer "F.Cu") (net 2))
 (segment (start 184.24375 104.43125) (end 182.2675 102.455) (width 0.2) (layer "F.Cu") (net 2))
 (segment (start 209.51975 94.27997) (end 198.64247 105.15725) (width 0.2) (layer "F.Cu") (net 2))
 (segment (start 157.534686 98.8735) (end 156.714 98.052814) (width 0.2) (layer "F.Cu") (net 2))
 (segment (start 186.860001 77.322501) (end 193.3575 83.82) (width 0.2) (layer "F.Cu") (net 11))
 (segment (start 158.115 78.4225) (end 159.214999 77.322501) (width 0.2) (layer "F.Cu") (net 11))
 (segment (start 159.214999 77.322501) (end 186.860001 77.322501) (width 0.2) (layer "F.Cu") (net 11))
 (segment (start 170.7045 84.883) (end 195.448126 84.883) (width 0.2) (layer "F.Cu") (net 12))
 (segment (start 195.448126 84.883) (end 195.7095 84.621626) (width 0.2) (layer "F.Cu") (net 12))
 (segment (start 195.7095 82.55437) (end 194.43513 81.28) (width 0.2) (layer "F.Cu") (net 12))
 (segment (start 194.43513 81.28) (end 193.3575 81.28) (width 0.2) (layer "F.Cu") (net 12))
 (segment (start 158.115 97.4725) (end 170.7045 84.883) (width 0.2) (layer "F.Cu") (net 12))
 (segment (start 195.7095 84.621626) (end 195.7095 82.55437) (width 0.2) (layer "F.Cu") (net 12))
 (segment (start 203.35875 87.66362) (end 203.35875 97.4725) (width 0.2) (layer "F.Cu") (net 13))
 (segment (start 194.43513 78.74) (end 203.35875 87.66362) (width 0.2) (layer "F.Cu") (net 13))
 (segment (start 193.3575 78.74) (end 194.43513 78.74) (width 0.2) (layer "F.Cu") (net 13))
 (segment (start 193.3575 76.2) (end 201.13625 76.2) (width 0.2) (layer "F.Cu") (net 14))
 (segment (start 201.13625 76.2) (end 203.35875 78.4225) (width 0.2) (layer "F.Cu") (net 14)))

